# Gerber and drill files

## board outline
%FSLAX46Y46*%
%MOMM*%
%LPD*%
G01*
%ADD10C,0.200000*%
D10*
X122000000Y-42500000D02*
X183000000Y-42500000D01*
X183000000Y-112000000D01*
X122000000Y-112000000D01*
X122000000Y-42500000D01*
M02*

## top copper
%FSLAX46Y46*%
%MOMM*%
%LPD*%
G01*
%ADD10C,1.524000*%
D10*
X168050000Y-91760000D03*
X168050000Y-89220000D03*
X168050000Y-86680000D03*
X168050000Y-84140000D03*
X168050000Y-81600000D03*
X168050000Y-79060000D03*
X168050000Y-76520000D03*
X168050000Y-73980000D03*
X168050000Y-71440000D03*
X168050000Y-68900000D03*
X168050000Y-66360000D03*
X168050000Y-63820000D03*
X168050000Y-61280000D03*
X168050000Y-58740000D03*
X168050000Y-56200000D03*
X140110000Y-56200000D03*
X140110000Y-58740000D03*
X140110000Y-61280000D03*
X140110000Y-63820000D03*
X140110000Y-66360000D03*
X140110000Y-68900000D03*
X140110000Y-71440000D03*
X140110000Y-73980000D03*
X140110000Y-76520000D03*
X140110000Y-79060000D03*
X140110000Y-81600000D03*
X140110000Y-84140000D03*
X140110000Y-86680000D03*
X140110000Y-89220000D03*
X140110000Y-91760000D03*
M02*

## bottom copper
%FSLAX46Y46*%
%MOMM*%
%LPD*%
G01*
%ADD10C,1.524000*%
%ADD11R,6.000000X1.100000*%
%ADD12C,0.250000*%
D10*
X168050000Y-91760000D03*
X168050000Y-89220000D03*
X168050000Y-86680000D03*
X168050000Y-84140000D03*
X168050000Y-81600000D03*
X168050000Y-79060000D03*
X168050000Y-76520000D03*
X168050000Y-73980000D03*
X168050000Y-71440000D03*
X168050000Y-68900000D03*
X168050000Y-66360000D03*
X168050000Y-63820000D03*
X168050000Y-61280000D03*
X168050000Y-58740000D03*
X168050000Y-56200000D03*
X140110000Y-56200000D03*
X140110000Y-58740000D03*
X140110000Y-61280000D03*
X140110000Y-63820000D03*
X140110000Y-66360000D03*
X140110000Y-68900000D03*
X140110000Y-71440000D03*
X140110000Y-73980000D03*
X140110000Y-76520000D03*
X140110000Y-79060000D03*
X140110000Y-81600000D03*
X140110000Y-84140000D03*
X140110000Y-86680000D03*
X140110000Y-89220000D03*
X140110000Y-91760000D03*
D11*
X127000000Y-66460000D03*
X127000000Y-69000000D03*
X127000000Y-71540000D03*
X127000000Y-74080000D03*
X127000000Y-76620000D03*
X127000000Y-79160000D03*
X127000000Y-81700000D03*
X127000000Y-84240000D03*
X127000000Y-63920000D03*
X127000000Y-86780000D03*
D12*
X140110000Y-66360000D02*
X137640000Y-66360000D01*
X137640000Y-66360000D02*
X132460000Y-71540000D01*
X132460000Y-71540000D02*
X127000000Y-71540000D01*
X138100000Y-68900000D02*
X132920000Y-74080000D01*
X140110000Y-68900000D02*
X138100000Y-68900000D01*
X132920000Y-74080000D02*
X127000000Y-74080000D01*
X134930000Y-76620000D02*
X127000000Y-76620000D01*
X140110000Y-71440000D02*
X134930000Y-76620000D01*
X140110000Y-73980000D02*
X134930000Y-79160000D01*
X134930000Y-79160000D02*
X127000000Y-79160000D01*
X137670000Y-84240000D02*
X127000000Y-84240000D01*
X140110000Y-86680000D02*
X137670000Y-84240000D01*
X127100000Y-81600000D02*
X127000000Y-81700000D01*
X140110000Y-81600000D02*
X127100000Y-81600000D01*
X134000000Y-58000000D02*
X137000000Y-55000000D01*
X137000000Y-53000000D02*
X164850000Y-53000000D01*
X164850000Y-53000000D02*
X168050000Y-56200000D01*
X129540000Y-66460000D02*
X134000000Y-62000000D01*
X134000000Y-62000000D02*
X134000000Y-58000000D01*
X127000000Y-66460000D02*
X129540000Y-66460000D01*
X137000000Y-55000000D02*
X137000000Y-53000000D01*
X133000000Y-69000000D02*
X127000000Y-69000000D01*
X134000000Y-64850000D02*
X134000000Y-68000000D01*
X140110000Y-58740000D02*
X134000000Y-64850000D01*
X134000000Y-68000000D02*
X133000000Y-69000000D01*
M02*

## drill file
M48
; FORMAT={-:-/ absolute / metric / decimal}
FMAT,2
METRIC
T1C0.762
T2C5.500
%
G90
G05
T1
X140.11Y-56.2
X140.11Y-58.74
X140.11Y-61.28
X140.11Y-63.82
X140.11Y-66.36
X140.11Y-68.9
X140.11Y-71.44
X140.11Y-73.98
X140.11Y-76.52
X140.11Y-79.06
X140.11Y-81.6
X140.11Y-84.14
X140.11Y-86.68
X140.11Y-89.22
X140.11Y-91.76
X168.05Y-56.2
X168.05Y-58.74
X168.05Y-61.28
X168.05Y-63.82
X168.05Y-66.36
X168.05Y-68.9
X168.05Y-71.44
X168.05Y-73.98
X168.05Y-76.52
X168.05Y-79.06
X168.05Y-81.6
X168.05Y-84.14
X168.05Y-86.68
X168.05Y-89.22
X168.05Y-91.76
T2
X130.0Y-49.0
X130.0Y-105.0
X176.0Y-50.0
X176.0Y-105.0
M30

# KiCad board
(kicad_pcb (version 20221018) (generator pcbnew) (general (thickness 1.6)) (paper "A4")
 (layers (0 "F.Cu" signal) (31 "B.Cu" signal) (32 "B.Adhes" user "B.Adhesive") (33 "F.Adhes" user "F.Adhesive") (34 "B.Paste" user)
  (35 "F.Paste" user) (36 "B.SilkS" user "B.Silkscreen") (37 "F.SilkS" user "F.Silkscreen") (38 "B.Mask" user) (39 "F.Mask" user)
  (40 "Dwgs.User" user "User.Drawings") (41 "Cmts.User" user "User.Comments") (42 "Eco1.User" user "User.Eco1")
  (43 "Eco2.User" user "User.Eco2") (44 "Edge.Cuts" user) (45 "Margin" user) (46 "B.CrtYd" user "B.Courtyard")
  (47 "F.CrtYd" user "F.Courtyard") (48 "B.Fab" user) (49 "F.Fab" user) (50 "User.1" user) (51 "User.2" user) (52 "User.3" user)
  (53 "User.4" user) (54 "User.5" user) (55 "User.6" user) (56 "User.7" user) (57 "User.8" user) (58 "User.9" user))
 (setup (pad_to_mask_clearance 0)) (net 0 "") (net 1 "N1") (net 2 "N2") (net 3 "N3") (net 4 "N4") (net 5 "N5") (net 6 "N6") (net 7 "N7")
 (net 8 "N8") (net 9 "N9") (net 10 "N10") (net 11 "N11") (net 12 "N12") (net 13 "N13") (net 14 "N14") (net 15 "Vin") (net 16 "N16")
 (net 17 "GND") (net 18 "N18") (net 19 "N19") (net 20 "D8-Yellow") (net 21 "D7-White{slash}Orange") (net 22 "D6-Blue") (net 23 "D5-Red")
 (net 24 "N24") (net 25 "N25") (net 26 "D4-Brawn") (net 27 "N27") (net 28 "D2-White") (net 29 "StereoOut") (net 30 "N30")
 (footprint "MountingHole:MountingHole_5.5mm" (layer "F.Cu") (at 130 49)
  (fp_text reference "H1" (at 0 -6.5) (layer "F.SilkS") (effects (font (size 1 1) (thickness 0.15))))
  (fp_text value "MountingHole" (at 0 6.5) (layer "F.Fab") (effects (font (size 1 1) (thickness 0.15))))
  (pad "" np_thru_hole circle (at 0 0) (size 5.5 5.5) (drill 5.5) (layers "*.Cu" "*.Mask")))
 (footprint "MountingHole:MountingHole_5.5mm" (layer "F.Cu") (at 176 105)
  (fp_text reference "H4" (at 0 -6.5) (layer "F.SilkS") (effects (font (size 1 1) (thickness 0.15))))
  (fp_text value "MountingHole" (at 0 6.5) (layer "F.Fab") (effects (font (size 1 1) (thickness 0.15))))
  (pad "" np_thru_hole circle (at 0 0) (size 5.5 5.5) (drill 5.5) (layers "*.Cu" "*.Mask")))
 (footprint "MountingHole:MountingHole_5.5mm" (layer "F.Cu") (at 176 50)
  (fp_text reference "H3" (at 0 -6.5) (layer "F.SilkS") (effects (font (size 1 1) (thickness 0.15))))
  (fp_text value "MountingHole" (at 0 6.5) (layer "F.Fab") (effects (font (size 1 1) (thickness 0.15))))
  (pad "" np_thru_hole circle (at 0 0) (size 5.5 5.5) (drill 5.5) (layers "*.Cu" "*.Mask")))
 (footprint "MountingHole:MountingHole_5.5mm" (layer "F.Cu") (at 130 105)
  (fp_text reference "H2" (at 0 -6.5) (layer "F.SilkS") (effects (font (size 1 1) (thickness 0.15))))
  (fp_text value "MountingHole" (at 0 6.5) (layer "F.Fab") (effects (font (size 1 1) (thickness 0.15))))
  (pad "" np_thru_hole circle (at 0 0) (size 5.5 5.5) (drill 5.5) (layers "*.Cu" "*.Mask")))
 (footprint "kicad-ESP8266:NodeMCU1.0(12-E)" (layer "F.Cu") (at 154.08 73.98 180)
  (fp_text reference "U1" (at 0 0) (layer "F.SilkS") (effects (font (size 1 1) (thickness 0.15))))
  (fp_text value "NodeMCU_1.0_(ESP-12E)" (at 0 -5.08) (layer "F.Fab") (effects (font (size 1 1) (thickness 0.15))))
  (pad "1" thru_hole circle (at -13.97 -17.78 180) (size 1.524 1.524) (drill 0.762) (layers "*.Cu" "*.Mask" "F.SilkS") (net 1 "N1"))
  (pad "2" thru_hole circle (at -13.97 -15.24 180) (size 1.524 1.524) (drill 0.762) (layers "*.Cu" "*.Mask" "F.SilkS") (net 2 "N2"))
  (pad "3" thru_hole circle (at -13.97 -12.7 180) (size 1.524 1.524) (drill 0.762) (layers "*.Cu" "*.Mask" "F.SilkS") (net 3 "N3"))
  (pad "4" thru_hole circle (at -13.97 -10.16 180) (size 1.524 1.524) (drill 0.762) (layers "*.Cu" "*.Mask" "F.SilkS") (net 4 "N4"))
  (pad "5" thru_hole circle (at -13.97 -7.62 180) (size 1.524 1.524) (drill 0.762) (layers "*.Cu" "*.Mask" "F.SilkS") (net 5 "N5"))
  (pad "6" thru_hole circle (at -13.97 -5.08 180) (size 1.524 1.524) (drill 0.762) (layers "*.Cu" "*.Mask" "F.SilkS") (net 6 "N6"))
  (pad "7" thru_hole circle (at -13.97 -2.54 180) (size 1.524 1.524) (drill 0.762) (layers "*.Cu" "*.Mask" "F.SilkS") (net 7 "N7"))
  (pad "8" thru_hole circle (at -13.97 0 180) (size 1.524 1.524) (drill 0.762) (layers "*.Cu" "*.Mask" "F.SilkS") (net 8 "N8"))
  (pad "9" thru_hole circle (at -13.97 2.54 180) (size 1.524 1.524) (drill 0.762) (layers "*.Cu" "*.Mask" "F.SilkS") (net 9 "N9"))
  (pad "10" thru_hole circle (at -13.97 5.08 180) (size 1.524 1.524) (drill 0.762) (layers "*.Cu" "*.Mask" "F.SilkS") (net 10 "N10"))
  (pad "11" thru_hole circle (at -13.97 7.62 180) (size 1.524 1.524) (drill 0.762) (layers "*.Cu" "*.Mask" "F.SilkS") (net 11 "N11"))
  (pad "12" thru_hole circle (at -13.97 10.16 180) (size 1.524 1.524) (drill 0.762) (layers "*.Cu" "*.Mask" "F.SilkS") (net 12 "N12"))
  (pad "13" thru_hole circle (at -13.97 12.7 180) (size 1.524 1.524) (drill 0.762) (layers "*.Cu" "*.Mask" "F.SilkS") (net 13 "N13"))
  (pad "14" thru_hole circle (at -13.97 15.24 180) (size 1.524 1.524) (drill 0.762) (layers "*.Cu" "*.Mask" "F.SilkS") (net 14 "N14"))
  (pad "15" thru_hole circle (at -13.97 17.78 180) (size 1.524 1.524) (drill 0.762) (layers "*.Cu" "*.Mask" "F.SilkS") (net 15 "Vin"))
  (pad "16" thru_hole circle (at 13.97 17.78 180) (size 1.524 1.524) (drill 0.762) (layers "*.Cu" "*.Mask" "F.SilkS") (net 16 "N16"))
  (pad "17" thru_hole circle (at 13.97 15.24 180) (size 1.524 1.524) (drill 0.762) (layers "*.Cu" "*.Mask" "F.SilkS") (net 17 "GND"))
  (pad "18" thru_hole circle (at 13.97 12.7 180) (size 1.524 1.524) (drill 0.762) (layers "*.Cu" "*.Mask" "F.SilkS") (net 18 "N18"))
  (pad "19" thru_hole circle (at 13.97 10.16 180) (size 1.524 1.524) (drill 0.762) (layers "*.Cu" "*.Mask" "F.SilkS") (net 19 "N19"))
  (pad "20" thru_hole circle (at 13.97 7.62 180) (size 1.524 1.524) (drill 0.762) (layers "*.Cu" "*.Mask" "F.SilkS") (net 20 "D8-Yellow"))
  (pad "21" thru_hole circle (at 13.97 5.08 180) (size 1.524 1.524) (drill 0.762) (layers "*.Cu" "*.Mask" "F.SilkS")
   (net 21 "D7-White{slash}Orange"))
  (pad "22" thru_hole circle (at 13.97 2.54 180) (size 1.524 1.524) (drill 0.762) (layers "*.Cu" "*.Mask" "F.SilkS") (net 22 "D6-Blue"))
  (pad "23" thru_hole circle (at 13.97 0 180) (size 1.524 1.524) (drill 0.762) (layers "*.Cu" "*.Mask" "F.SilkS") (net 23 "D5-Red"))
  (pad "24" thru_hole circle (at 13.97 -2.54 180) (size 1.524 1.524) (drill 0.762) (layers "*.Cu" "*.Mask" "F.SilkS") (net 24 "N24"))
  (pad "25" thru_hole circle (at 13.97 -5.08 180) (size 1.524 1.524) (drill 0.762) (layers "*.Cu" "*.Mask" "F.SilkS") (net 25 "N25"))
  (pad "26" thru_hole circle (at 13.97 -7.62 180) (size 1.524 1.524) (drill 0.762) (layers "*.Cu" "*.Mask" "F.SilkS") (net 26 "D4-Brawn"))
  (pad "27" thru_hole circle (at 13.97 -10.16 180) (size 1.524 1.524) (drill 0.762) (layers "*.Cu" "*.Mask" "F.SilkS") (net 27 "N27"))
  (pad "28" thru_hole circle (at 13.97 -12.7 180) (size 1.524 1.524) (drill 0.762) (layers "*.Cu" "*.Mask" "F.SilkS") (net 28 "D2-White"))
  (pad "29" thru_hole circle (at 13.97 -15.24 180) (size 1.524 1.524) (drill 0.762) (layers "*.Cu" "*.Mask" "F.SilkS") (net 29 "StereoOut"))
  (pad "30" thru_hole circle (at 13.97 -17.78 180) (size 1.524 1.524) (drill 0.762) (layers "*.Cu" "*.Mask" "F.SilkS") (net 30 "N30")))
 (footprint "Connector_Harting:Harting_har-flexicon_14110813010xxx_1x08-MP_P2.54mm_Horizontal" (layer "B.Cu") (at 128.3 75.35 -90)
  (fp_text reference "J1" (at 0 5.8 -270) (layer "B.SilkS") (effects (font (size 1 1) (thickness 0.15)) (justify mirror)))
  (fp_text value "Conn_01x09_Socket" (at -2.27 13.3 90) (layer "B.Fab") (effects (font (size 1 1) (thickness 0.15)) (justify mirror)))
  (pad "1" smd rect (at -8.89 1.3 270) (size 1.1 6) (layers "B.Cu" "B.Paste" "B.Mask") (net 15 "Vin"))
  (pad "2" smd rect (at -6.35 1.3 270) (size 1.1 6) (layers "B.Cu" "B.Paste" "B.Mask") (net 17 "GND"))
  (pad "3" smd rect (at -3.81 1.3 270) (size 1.1 6) (layers "B.Cu" "B.Paste" "B.Mask") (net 20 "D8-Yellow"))
  (pad "4" smd rect (at -1.27 1.3 270) (size 1.1 6) (layers "B.Cu" "B.Paste" "B.Mask") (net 21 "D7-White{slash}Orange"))
  (pad "5" smd rect (at 1.27 1.3 270) (size 1.1 6) (layers "B.Cu" "B.Paste" "B.Mask") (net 22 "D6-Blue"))
  (pad "6" smd rect (at 3.81 1.3 270) (size 1.1 6) (layers "B.Cu" "B.Paste" "B.Mask") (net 23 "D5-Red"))
  (pad "7" smd rect (at 6.35 1.3 270) (size 1.1 6) (layers "B.Cu" "B.Paste" "B.Mask") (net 26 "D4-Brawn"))
  (pad "8" smd rect (at 8.89 1.3 270) (size 1.1 6) (layers "B.Cu" "B.Paste" "B.Mask") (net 28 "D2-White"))
  (pad "MP" smd rect (at -11.43 1.3 270) (size 1.1 6) (layers "B.Cu" "B.Paste" "B.Mask"))
  (pad "MP" smd rect (at 11.43 1.3 270) (size 1.1 6) (layers "B.Cu" "B.Paste" "B.Mask")))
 (gr_rect (start 122 42.5) (end 183 112) (stroke (width 0.2) (type default)) (fill none) (layer "Edge.Cuts"))
 (segment (start 140.11 66.36) (end 137.64 66.36) (width 0.25) (layer "B.Cu") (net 20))
 (segment (start 137.64 66.36) (end 132.46 71.54) (width 0.25) (layer "B.Cu") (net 20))
 (segment (start 132.46 71.54) (end 127 71.54) (width 0.25) (layer "B.Cu") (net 20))
 (segment (start 138.1 68.9) (end 132.92 74.08) (width 0.25) (layer "B.Cu") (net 21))
 (segment (start 140.11 68.9) (end 138.1 68.9) (width 0.25) (layer "B.Cu") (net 21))
 (segment (start 132.92 74.08) (end 127 74.08) (width 0.25) (layer "B.Cu") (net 21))
 (segment (start 134.93 76.62) (end 127 76.62) (width 0.25) (layer "B.Cu") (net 22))
 (segment (start 140.11 71.44) (end 134.93 76.62) (width 0.25) (layer "B.Cu") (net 22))
 (segment (start 140.11 73.98) (end 134.93 79.16) (width 0.25) (layer "B.Cu") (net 23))
 (segment (start 134.93 79.16) (end 127 79.16) (width 0.25) (layer "B.Cu") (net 23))
 (segment (start 137.67 84.24) (end 127 84.24) (width 0.25) (layer "B.Cu") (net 28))
 (segment (start 140.11 86.68) (end 137.67 84.24) (width 0.25) (layer "B.Cu") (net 28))
 (segment (start 127.1 81.6) (end 127 81.7) (width 0.25) (layer "B.Cu") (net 26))
 (segment (start 140.11 81.6) (end 127.1 81.6) (width 0.25) (layer "B.Cu") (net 26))
 (segment (start 134 58) (end 137 55) (width 0.25) (layer "B.Cu") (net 15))
 (segment (start 137 53) (end 164.85 53) (width 0.25) (layer "B.Cu") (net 15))
 (segment (start 164.85 53) (end 168.05 56.2) (width 0.25) (layer "B.Cu") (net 15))
 (segment (start 129.54 66.46) (end 134 62) (width 0.25) (layer "B.Cu") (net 15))
 (segment (start 134 62) (end 134 58) (width 0.25) (layer "B.Cu") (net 15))
 (segment (start 127 66.46) (end 129.54 66.46) (width 0.25) (layer "B.Cu") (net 15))
 (segment (start 137 55) (end 137 53) (width 0.25) (layer "B.Cu") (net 15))
 (segment (start 133 69) (end 127 69) (width 0.25) (layer "B.Cu") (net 17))
 (segment (start 134 64.85) (end 134 68) (width 0.25) (layer "B.Cu") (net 17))
 (segment (start 140.11 58.74) (end 134 64.85) (width 0.25) (layer "B.Cu") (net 17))
 (segment (start 134 68) (end 133 69) (width 0.25) (layer "B.Cu") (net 17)))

